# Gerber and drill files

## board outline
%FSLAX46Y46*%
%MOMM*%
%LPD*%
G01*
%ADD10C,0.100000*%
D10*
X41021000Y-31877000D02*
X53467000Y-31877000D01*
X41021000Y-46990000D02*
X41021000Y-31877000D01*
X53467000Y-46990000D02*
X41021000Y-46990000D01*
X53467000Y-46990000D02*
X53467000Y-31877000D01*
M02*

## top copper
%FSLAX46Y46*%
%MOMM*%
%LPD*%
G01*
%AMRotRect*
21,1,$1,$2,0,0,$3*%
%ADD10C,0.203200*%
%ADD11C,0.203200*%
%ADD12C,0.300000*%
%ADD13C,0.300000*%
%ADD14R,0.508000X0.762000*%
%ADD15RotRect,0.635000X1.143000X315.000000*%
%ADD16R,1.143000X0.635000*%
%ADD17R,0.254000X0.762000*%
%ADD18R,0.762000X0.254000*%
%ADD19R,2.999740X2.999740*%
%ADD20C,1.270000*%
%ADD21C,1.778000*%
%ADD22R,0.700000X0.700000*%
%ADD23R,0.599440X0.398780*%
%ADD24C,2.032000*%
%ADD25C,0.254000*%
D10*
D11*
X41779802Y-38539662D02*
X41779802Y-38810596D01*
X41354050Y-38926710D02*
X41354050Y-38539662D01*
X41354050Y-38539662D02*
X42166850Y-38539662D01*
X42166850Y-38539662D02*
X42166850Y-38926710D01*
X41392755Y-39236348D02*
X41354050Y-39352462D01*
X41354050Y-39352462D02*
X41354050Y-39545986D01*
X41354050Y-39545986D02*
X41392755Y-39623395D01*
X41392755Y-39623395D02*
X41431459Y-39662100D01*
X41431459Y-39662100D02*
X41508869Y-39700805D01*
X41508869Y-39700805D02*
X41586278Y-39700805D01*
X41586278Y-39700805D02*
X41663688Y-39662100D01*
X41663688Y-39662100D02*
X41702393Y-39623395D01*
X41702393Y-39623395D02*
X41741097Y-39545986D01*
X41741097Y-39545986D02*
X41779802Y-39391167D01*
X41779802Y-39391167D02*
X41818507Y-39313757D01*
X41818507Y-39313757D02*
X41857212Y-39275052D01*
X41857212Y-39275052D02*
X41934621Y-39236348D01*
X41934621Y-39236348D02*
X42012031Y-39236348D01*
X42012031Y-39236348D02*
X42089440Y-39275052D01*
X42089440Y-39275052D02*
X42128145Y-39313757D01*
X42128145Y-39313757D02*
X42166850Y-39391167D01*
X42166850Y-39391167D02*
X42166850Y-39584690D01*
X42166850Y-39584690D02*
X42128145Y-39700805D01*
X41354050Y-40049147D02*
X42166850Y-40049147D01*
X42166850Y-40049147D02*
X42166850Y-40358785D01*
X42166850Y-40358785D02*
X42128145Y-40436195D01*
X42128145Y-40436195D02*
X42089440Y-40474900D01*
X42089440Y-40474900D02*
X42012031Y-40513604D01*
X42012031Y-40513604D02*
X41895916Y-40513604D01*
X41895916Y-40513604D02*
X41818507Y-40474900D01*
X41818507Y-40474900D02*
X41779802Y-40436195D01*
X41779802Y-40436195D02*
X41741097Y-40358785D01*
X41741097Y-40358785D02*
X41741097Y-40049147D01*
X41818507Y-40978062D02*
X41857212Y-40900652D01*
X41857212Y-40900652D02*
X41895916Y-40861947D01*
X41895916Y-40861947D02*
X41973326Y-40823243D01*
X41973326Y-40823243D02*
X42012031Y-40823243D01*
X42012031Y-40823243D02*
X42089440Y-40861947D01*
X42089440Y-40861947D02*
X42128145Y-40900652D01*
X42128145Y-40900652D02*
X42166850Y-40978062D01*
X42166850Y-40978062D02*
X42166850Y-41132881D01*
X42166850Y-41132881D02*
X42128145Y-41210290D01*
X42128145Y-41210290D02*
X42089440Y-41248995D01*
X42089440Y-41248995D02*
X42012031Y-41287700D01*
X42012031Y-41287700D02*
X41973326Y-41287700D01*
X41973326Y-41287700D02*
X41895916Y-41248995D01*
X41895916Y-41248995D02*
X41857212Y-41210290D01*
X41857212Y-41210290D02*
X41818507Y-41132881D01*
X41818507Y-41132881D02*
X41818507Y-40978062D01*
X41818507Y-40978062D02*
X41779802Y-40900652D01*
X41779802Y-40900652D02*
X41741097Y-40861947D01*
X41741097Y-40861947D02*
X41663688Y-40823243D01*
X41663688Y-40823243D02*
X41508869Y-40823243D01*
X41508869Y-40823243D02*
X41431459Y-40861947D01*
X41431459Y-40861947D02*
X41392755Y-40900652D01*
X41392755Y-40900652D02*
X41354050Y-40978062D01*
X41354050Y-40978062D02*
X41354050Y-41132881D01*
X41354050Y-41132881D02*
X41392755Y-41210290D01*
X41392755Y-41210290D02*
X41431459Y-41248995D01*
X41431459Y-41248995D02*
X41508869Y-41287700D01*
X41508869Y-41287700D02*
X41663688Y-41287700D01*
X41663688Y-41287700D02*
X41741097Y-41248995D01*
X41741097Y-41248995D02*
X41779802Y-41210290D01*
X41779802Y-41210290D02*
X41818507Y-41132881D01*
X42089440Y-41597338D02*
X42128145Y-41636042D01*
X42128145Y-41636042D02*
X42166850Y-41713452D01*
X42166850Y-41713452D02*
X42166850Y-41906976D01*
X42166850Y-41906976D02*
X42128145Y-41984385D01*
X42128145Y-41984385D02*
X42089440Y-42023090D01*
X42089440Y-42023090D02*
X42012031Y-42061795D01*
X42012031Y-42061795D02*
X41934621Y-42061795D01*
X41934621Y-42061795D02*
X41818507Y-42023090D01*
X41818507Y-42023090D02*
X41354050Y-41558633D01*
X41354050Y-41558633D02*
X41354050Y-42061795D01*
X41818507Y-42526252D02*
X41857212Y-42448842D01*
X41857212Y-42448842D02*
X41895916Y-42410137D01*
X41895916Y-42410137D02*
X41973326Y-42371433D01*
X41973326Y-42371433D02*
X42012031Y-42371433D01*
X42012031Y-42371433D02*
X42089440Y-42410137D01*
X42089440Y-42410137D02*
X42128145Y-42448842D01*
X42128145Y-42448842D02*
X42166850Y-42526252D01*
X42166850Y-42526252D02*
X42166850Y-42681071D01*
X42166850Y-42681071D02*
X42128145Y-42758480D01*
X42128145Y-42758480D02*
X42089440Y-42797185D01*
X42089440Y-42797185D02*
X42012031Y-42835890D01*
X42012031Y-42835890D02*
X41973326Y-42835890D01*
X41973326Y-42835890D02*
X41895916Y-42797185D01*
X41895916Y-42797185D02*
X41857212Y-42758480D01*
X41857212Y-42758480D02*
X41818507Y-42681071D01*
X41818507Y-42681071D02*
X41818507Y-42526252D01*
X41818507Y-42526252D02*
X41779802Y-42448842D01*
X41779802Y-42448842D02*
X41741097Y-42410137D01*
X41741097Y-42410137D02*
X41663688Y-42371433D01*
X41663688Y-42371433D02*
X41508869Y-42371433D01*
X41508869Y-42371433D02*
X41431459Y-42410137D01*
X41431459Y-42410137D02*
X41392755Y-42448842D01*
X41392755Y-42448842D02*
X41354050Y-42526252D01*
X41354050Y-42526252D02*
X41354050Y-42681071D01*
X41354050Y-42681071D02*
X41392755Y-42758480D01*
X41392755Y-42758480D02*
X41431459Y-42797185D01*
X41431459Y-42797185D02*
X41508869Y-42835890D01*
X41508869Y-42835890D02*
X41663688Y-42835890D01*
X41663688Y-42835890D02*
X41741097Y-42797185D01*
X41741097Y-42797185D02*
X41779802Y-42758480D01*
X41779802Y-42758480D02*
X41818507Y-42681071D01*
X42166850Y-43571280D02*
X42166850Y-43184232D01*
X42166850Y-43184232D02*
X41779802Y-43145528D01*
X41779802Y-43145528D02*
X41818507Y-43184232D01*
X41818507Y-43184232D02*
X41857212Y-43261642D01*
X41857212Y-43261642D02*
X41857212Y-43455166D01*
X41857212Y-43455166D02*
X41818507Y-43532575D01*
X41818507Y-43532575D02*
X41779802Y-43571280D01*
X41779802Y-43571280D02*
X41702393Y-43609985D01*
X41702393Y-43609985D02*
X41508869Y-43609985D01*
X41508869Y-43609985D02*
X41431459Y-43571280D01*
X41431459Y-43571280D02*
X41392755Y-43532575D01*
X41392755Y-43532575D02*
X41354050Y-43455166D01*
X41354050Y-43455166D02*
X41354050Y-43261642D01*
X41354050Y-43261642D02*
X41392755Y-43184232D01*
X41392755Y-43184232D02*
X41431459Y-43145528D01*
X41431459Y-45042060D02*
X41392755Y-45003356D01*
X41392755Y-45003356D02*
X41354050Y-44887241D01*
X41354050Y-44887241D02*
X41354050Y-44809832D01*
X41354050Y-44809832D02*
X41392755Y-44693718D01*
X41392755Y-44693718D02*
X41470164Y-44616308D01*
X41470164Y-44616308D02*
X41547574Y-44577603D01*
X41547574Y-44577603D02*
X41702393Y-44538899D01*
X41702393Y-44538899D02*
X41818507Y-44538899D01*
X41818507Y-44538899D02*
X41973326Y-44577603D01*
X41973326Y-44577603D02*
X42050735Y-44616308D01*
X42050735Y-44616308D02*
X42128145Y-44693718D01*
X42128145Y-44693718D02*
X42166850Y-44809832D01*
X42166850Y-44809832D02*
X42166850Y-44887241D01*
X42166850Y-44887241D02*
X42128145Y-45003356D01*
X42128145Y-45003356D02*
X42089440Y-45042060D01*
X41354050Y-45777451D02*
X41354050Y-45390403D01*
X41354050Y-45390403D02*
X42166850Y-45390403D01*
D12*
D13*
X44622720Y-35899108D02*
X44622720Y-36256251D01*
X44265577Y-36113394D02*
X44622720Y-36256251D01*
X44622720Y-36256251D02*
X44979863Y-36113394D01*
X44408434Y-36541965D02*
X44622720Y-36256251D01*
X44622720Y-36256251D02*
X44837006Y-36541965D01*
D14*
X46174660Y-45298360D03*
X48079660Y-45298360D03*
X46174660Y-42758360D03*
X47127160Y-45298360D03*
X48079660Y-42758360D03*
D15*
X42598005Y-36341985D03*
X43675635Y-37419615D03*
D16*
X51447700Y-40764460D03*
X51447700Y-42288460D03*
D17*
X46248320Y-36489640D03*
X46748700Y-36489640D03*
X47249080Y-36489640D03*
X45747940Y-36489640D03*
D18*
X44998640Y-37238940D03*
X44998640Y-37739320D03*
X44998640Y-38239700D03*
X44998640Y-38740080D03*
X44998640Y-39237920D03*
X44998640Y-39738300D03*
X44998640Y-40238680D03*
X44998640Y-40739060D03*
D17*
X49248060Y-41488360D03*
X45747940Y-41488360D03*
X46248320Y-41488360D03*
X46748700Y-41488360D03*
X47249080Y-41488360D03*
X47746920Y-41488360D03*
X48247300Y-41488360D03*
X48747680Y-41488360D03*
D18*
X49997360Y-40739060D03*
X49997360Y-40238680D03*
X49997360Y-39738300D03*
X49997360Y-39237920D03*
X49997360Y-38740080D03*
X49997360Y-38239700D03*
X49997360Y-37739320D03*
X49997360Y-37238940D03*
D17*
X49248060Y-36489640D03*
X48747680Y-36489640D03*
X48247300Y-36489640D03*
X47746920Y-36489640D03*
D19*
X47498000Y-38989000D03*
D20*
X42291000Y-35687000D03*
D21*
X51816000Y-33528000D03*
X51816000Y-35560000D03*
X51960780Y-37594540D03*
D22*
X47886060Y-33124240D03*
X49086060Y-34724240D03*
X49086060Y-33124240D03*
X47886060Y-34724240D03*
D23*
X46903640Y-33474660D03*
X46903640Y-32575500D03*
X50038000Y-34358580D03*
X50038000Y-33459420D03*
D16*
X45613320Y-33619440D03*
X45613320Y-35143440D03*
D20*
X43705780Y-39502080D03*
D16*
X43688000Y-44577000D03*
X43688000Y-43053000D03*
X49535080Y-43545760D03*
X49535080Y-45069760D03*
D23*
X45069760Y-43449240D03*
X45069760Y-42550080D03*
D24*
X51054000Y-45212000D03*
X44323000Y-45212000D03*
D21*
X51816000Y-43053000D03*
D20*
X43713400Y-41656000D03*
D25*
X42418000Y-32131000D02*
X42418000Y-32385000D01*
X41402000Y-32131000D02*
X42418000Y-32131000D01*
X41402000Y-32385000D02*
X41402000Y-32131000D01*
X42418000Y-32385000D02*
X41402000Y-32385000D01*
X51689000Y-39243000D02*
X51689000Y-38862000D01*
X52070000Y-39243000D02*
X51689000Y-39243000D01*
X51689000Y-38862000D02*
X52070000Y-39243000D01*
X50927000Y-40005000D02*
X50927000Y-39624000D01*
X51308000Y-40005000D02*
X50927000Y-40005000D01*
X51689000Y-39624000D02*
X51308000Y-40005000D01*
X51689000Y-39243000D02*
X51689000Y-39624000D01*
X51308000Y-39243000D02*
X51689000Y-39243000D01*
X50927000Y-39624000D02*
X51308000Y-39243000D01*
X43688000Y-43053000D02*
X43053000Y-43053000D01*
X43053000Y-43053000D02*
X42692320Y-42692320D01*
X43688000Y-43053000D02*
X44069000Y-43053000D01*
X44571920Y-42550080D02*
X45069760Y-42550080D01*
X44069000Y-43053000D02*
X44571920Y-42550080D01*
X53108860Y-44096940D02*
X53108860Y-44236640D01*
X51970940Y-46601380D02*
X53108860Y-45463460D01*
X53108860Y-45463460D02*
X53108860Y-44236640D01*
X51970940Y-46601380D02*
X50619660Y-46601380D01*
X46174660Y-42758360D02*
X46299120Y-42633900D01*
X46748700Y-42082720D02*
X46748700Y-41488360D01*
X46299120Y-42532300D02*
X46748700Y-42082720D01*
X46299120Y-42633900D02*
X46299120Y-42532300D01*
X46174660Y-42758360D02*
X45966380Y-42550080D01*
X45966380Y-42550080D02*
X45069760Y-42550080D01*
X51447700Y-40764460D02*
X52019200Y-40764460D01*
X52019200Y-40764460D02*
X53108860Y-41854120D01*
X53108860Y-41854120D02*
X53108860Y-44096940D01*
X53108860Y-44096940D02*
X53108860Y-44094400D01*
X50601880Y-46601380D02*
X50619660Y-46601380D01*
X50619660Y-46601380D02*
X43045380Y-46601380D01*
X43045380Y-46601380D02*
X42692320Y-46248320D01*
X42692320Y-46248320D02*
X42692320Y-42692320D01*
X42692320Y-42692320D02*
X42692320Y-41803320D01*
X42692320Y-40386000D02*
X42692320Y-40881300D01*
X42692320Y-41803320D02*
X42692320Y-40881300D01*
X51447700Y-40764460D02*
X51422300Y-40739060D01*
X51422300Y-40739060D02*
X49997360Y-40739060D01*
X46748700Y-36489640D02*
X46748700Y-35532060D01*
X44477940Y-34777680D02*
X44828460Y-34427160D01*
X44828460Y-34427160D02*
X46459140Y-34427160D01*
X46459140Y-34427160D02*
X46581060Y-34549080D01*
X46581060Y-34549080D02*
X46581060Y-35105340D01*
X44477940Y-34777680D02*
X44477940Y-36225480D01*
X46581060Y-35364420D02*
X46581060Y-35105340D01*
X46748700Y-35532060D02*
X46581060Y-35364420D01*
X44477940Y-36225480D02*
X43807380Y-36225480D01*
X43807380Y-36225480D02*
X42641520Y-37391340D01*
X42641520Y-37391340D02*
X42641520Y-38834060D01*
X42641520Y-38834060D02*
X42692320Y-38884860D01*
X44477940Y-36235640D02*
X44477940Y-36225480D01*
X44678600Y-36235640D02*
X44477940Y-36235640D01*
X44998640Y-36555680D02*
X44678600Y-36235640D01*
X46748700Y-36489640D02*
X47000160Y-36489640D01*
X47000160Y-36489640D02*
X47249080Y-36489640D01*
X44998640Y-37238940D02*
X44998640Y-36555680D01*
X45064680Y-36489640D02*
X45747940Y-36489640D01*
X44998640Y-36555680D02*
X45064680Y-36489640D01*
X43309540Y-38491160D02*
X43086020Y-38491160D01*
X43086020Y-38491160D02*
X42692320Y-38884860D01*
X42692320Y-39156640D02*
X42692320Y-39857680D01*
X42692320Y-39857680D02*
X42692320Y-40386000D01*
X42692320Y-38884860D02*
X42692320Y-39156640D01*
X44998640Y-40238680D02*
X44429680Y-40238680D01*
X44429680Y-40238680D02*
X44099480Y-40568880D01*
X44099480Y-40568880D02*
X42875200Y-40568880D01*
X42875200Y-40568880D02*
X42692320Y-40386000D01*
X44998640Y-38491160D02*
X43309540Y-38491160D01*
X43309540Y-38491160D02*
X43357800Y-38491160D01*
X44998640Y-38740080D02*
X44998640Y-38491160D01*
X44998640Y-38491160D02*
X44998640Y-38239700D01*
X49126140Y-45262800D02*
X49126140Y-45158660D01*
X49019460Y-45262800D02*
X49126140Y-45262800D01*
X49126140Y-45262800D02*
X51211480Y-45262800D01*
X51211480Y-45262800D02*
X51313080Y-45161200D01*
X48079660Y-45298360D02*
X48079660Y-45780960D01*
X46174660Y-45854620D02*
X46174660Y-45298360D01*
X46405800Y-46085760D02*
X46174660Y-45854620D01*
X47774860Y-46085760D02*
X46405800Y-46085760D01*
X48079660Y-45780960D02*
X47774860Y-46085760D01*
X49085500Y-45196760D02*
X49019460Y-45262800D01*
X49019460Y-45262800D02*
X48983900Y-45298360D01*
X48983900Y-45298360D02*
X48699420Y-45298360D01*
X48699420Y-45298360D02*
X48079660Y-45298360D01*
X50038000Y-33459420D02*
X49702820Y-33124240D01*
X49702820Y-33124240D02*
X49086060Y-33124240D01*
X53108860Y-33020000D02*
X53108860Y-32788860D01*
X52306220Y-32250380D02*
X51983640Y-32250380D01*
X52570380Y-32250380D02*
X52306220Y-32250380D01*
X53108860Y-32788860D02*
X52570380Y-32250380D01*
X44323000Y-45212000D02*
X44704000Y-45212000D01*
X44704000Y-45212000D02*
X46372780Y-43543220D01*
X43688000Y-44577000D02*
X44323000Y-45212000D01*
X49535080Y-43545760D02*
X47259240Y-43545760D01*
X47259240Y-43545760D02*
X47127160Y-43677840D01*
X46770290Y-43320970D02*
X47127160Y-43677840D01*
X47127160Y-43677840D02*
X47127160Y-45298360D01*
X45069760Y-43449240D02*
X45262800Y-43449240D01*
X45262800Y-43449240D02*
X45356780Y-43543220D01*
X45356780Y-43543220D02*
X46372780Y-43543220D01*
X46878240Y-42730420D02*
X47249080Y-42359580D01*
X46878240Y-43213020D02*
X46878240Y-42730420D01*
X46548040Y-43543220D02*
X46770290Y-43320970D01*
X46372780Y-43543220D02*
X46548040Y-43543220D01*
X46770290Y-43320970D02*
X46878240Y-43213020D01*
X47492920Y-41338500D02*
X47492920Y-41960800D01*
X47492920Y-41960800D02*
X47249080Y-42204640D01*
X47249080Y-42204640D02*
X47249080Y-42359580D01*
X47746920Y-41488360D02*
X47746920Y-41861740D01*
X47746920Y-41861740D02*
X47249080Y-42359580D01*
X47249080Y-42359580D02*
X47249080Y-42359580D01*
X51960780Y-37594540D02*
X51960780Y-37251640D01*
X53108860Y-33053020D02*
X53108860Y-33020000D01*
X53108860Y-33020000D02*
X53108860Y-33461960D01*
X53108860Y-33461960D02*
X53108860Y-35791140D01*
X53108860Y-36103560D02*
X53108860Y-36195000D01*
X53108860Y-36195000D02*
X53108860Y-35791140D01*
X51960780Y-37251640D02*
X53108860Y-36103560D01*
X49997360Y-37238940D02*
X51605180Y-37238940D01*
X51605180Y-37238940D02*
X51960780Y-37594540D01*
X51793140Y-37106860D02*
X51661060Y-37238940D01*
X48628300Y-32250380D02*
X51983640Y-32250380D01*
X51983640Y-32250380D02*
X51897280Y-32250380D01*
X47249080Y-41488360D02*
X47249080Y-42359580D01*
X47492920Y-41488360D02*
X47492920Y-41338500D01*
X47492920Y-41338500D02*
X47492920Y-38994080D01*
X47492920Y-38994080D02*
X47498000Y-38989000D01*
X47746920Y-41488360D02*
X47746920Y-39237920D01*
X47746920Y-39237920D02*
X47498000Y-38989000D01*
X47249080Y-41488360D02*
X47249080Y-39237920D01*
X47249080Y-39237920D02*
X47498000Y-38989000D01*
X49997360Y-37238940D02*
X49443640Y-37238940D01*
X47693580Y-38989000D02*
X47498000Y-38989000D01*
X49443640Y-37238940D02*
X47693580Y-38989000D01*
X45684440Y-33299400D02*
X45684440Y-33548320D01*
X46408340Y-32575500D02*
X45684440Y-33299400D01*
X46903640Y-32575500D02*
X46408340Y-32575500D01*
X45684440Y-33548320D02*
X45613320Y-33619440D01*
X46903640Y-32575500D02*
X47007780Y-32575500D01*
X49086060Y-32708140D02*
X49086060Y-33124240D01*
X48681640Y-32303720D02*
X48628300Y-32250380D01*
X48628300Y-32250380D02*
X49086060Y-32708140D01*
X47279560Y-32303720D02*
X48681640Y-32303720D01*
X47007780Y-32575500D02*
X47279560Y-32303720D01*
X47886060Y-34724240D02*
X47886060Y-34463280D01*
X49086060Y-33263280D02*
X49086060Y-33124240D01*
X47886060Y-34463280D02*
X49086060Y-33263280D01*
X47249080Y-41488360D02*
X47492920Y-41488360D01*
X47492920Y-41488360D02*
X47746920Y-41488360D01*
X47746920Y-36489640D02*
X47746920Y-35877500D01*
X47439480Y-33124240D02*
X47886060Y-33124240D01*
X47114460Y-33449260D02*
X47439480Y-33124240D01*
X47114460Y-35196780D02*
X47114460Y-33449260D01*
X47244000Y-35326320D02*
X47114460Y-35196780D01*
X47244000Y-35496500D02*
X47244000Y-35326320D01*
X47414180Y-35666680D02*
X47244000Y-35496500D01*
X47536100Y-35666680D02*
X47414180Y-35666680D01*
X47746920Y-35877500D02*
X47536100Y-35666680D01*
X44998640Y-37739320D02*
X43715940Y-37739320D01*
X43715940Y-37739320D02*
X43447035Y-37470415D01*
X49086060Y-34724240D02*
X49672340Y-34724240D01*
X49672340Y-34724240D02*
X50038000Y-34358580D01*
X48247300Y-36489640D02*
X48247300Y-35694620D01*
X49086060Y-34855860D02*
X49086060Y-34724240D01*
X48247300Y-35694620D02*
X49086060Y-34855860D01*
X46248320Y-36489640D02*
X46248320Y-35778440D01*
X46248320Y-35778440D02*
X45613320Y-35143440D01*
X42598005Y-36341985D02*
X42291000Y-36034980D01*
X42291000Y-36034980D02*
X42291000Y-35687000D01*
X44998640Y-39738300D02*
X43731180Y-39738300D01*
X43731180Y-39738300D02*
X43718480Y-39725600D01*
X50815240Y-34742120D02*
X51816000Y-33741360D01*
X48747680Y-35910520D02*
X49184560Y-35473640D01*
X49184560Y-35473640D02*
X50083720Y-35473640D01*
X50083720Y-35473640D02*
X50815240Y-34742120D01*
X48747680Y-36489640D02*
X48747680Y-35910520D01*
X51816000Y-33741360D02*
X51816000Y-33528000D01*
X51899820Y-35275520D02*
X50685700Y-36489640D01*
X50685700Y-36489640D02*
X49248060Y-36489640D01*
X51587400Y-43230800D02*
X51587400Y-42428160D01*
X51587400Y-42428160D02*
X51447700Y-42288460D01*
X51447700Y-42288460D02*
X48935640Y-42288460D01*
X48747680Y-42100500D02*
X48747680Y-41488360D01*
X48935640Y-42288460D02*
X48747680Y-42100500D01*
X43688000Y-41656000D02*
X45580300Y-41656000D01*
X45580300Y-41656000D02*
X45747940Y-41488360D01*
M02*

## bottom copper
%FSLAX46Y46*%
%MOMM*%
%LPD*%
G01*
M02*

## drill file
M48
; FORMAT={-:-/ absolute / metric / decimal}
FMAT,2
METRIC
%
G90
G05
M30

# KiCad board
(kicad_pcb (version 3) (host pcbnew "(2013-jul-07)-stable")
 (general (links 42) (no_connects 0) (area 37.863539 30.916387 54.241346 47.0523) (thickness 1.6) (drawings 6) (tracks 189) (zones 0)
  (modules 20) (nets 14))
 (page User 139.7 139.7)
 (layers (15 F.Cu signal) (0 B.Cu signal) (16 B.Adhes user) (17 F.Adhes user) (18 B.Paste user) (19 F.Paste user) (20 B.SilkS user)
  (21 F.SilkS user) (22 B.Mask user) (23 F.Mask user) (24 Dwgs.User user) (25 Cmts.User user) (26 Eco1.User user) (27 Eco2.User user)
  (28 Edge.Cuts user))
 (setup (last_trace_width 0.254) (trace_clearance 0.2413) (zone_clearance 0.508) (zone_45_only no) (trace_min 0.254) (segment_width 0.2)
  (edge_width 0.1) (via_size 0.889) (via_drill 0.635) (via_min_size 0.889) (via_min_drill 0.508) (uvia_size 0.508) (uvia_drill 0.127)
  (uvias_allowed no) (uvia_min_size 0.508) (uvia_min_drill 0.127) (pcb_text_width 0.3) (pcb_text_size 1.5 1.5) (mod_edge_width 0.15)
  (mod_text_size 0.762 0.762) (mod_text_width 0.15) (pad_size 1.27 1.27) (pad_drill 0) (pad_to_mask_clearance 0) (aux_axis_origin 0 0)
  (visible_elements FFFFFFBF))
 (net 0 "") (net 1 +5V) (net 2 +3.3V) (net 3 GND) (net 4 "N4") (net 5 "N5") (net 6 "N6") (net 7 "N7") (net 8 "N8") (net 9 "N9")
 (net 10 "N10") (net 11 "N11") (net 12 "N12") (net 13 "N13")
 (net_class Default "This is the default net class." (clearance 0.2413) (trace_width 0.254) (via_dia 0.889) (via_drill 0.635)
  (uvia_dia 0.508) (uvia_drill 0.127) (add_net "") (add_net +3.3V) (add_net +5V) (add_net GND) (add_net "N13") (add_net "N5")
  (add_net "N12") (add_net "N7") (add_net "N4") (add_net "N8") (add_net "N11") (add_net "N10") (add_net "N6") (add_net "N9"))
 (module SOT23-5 (layer F.Cu) (at 47.12716 44.02836)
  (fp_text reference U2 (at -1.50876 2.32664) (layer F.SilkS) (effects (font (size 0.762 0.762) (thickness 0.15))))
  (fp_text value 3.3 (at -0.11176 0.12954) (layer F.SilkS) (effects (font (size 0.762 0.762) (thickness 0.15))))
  (pad 1 smd rect (at -0.9525 1.27) (size 0.508 0.762) (layers F.Cu F.Paste F.Mask) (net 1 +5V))
  (pad 3 smd rect (at 0.9525 1.27) (size 0.508 0.762) (layers F.Cu F.Paste F.Mask) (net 1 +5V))
  (pad 5 smd rect (at -0.9525 -1.27) (size 0.508 0.762) (layers F.Cu F.Paste F.Mask) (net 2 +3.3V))
  (pad 2 smd rect (at 0 1.27) (size 0.508 0.762) (layers F.Cu F.Paste F.Mask) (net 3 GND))
  (pad 4 smd rect (at 0.9525 -1.27) (size 0.508 0.762) (layers F.Cu F.Paste F.Mask)))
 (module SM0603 (layer F.Cu) (at 43.13682 36.8808 315)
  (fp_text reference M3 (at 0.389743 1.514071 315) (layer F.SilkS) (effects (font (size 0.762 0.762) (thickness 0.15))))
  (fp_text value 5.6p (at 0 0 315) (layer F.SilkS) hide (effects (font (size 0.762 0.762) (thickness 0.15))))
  (pad 1 smd rect (at -0.762 0 315) (size 0.635 1.143) (layers F.Cu F.Paste F.Mask) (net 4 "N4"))
  (pad 2 smd rect (at 0.762 0 315) (size 0.635 1.143) (layers F.Cu F.Paste F.Mask) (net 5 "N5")))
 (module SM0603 (layer F.Cu) (at 51.4477 41.52646 270)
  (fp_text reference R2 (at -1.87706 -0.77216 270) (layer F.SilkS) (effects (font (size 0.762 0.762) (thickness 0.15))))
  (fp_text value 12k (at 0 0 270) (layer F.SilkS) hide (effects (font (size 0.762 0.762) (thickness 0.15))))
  (pad 1 smd rect (at -0.762 0 270) (size 0.635 1.143) (layers F.Cu F.Paste F.Mask) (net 2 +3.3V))
  (pad 2 smd rect (at 0.762 0 270) (size 0.635 1.143) (layers F.Cu F.Paste F.Mask) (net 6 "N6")))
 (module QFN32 (layer F.Cu) (at 47.498 38.989)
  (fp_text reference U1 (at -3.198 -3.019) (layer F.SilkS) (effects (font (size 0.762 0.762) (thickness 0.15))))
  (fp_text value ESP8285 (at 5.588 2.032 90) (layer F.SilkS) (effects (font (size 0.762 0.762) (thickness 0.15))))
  (pad 31 smd rect (at -1.24968 -2.49936) (size 0.254 0.762) (layers F.Cu F.Paste F.Mask) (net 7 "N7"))
  (pad 30 smd rect (at -0.7493 -2.49936) (size 0.254 0.762) (layers F.Cu F.Paste F.Mask) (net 2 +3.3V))
  (pad 29 smd rect (at -0.24892 -2.49936) (size 0.254 0.762) (layers F.Cu F.Paste F.Mask) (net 2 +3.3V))
  (pad 32 smd rect (at -1.75006 -2.49936) (size 0.254 0.762) (layers F.Cu F.Paste F.Mask) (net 2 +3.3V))
  (pad 1 smd rect (at -2.49936 -1.75006 90) (size 0.254 0.762) (layers F.Cu F.Paste F.Mask) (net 2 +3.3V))
  (pad 2 smd rect (at -2.49936 -1.24968 90) (size 0.254 0.762) (layers F.Cu F.Paste F.Mask) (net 5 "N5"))
  (pad 3 smd rect (at -2.49936 -0.7493 90) (size 0.254 0.762) (layers F.Cu F.Paste F.Mask) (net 2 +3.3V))
  (pad 4 smd rect (at -2.49936 -0.24892 90) (size 0.254 0.762) (layers F.Cu F.Paste F.Mask) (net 2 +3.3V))
  (pad 5 smd rect (at -2.49936 0.24892 90) (size 0.254 0.762) (layers F.Cu F.Paste F.Mask))
  (pad 6 smd rect (at -2.49936 0.7493 90) (size 0.254 0.762) (layers F.Cu F.Paste F.Mask) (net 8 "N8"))
  (pad 7 smd rect (at -2.49936 1.24968 90) (size 0.254 0.762) (layers F.Cu F.Paste F.Mask) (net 2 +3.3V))
  (pad 8 smd rect (at -2.49936 1.75006 90) (size 0.254 0.762) (layers F.Cu F.Paste F.Mask))
  (pad 16 smd rect (at 1.75006 2.49936) (size 0.254 0.762) (layers F.Cu F.Paste F.Mask))
  (pad 9 smd rect (at -1.75006 2.49936) (size 0.254 0.762) (layers F.Cu F.Paste F.Mask) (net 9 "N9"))
  (pad 10 smd rect (at -1.24968 2.49936) (size 0.254 0.762) (layers F.Cu F.Paste F.Mask))
  (pad 11 smd rect (at -0.7493 2.49936) (size 0.254 0.762) (layers F.Cu F.Paste F.Mask) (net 2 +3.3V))
  (pad 12 smd rect (at -0.24892 2.49936) (size 0.254 0.762) (layers F.Cu F.Paste F.Mask) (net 3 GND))
  (pad 13 smd rect (at 0.24892 2.49936) (size 0.254 0.762) (layers F.Cu F.Paste F.Mask) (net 3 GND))
  (pad 14 smd rect (at 0.7493 2.49936) (size 0.254 0.762) (layers F.Cu F.Paste F.Mask))
  (pad 15 smd rect (at 1.24968 2.49936) (size 0.254 0.762) (layers F.Cu F.Paste F.Mask) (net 6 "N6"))
  (pad 17 smd rect (at 2.49936 1.75006 90) (size 0.254 0.762) (layers F.Cu F.Paste F.Mask) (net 2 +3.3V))
  (pad 18 smd rect (at 2.49936 1.24968 90) (size 0.254 0.762) (layers F.Cu F.Paste F.Mask))
  (pad 19 smd rect (at 2.49936 0.7493 90) (size 0.254 0.762) (layers F.Cu F.Paste F.Mask))
  (pad 20 smd rect (at 2.49936 0.24892 90) (size 0.254 0.762) (layers F.Cu F.Paste F.Mask))
  (pad 21 smd rect (at 2.49936 -0.24892 90) (size 0.254 0.762) (layers F.Cu F.Paste F.Mask))
  (pad 22 smd rect (at 2.49936 -0.7493 90) (size 0.254 0.762) (layers F.Cu F.Paste F.Mask))
  (pad 23 smd rect (at 2.49936 -1.24968 90) (size 0.254 0.762) (layers F.Cu F.Paste F.Mask))
  (pad 24 smd rect (at 2.49936 -1.75006 90) (size 0.254 0.762) (layers F.Cu F.Paste F.Mask) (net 3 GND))
  (pad 25 smd rect (at 1.75006 -2.49936) (size 0.254 0.762) (layers F.Cu F.Paste F.Mask) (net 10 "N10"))
  (pad 26 smd rect (at 1.24968 -2.49936) (size 0.254 0.762) (layers F.Cu F.Paste F.Mask) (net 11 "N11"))
  (pad 27 smd rect (at 0.7493 -2.49936) (size 0.254 0.762) (layers F.Cu F.Paste F.Mask) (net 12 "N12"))
  (pad 28 smd rect (at 0.24892 -2.49936) (size 0.254 0.762) (layers F.Cu F.Paste F.Mask) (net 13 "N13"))
  (pad 33 smd rect (at 0 0) (size 2.99974 2.99974) (layers F.Cu F.Paste F.Mask) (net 3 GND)))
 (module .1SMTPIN (layer F.Cu) (at 42.291 35.687)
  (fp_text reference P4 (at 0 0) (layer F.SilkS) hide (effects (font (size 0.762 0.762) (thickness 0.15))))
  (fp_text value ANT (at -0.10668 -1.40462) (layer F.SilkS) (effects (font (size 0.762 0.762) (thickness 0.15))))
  (pad 1 smd circle (at 0 0) (size 1.27 1.27) (layers F.Cu F.Paste F.Mask) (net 4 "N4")))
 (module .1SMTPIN (layer F.Cu) (at 51.816 33.528)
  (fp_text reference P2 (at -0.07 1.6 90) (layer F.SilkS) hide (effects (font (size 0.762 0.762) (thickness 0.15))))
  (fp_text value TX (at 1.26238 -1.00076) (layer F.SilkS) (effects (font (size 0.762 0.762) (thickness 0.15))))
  (pad 1 smd circle (at 0 0) (size 1.778 1.778) (layers F.Cu F.Paste F.Mask) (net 11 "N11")))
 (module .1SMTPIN (layer F.Cu) (at 51.816 35.56)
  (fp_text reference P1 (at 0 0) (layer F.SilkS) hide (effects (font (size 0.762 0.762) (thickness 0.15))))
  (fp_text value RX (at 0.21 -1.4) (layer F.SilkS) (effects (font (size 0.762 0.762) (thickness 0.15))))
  (pad 1 smd circle (at 0 0) (size 1.778 1.778) (layers F.Cu F.Paste F.Mask) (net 10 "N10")))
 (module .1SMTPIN (layer F.Cu) (at 51.96078 37.59454)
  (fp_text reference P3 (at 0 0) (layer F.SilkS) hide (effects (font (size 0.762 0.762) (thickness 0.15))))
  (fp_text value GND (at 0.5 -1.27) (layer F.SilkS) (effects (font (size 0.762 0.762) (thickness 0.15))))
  (pad 1 smd circle (at 0 0) (size 1.778 1.778) (layers F.Cu F.Paste F.Mask) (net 3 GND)))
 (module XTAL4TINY (layer F.Cu) (at 48.48606 33.92424 270)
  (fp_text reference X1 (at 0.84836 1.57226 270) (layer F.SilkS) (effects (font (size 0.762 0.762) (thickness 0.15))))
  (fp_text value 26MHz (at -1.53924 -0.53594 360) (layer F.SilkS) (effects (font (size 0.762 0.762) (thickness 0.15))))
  (pad 1 smd rect (at -0.8 0.6 270) (size 0.7 0.7) (layers F.Cu F.Paste F.Mask) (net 13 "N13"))
  (pad 2 smd rect (at 0.8 -0.6 270) (size 0.7 0.7) (layers F.Cu F.Paste F.Mask) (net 12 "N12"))
  (pad 3 smd rect (at -0.8 -0.6 270) (size 0.7 0.7) (layers F.Cu F.Paste F.Mask) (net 3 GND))
  (pad 4 smd rect (at 0.8 0.6 270) (size 0.7 0.7) (layers F.Cu F.Paste F.Mask) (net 3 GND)))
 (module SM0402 (layer F.Cu) (at 46.90364 33.02508 90)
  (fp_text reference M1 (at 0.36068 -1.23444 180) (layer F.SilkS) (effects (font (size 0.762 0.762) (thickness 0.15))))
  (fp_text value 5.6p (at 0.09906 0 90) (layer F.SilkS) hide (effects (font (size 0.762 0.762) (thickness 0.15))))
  (pad 1 smd rect (at -0.44958 0 90) (size 0.39878 0.59944) (layers F.Cu F.Paste F.Mask) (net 13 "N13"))
  (pad 2 smd rect (at 0.44958 0 90) (size 0.39878 0.59944) (layers F.Cu F.Paste F.Mask) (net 3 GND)))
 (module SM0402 (layer F.Cu) (at 50.038 33.909 90)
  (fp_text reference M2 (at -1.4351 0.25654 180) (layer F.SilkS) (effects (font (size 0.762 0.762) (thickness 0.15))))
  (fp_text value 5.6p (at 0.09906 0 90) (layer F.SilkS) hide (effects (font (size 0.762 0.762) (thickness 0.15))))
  (pad 1 smd rect (at -0.44958 0 90) (size 0.39878 0.59944) (layers F.Cu F.Paste F.Mask) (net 12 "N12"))
  (pad 2 smd rect (at 0.44958 0 90) (size 0.39878 0.59944) (layers F.Cu F.Paste F.Mask) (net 3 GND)))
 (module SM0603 (layer F.Cu) (at 45.61332 34.38144 270)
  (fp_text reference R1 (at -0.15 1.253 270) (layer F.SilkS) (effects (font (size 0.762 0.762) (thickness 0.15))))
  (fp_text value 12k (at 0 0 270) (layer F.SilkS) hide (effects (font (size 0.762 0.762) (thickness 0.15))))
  (pad 1 smd rect (at -0.762 0 270) (size 0.635 1.143) (layers F.Cu F.Paste F.Mask) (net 3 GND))
  (pad 2 smd rect (at 0.762 0 270) (size 0.635 1.143) (layers F.Cu F.Paste F.Mask) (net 7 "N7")))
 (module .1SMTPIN (layer F.Cu) (at 43.70324 39.50208)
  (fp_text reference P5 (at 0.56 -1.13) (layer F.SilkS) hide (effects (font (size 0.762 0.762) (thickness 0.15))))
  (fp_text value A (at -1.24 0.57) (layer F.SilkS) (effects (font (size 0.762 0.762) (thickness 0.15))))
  (pad 1 smd circle (at 0.00254 0) (size 1.27 1.27) (layers F.Cu F.Paste F.Mask) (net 8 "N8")))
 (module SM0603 (layer F.Cu) (at 43.688 43.815 90)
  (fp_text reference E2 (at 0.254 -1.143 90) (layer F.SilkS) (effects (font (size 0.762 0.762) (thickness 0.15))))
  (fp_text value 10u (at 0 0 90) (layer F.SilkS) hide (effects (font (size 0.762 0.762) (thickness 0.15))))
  (pad 1 smd rect (at -0.762 0 90) (size 0.635 1.143) (layers F.Cu F.Paste F.Mask) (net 3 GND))
  (pad 2 smd rect (at 0.762 0 90) (size 0.635 1.143) (layers F.Cu F.Paste F.Mask) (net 2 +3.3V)))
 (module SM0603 (layer F.Cu) (at 49.53508 44.30776 270)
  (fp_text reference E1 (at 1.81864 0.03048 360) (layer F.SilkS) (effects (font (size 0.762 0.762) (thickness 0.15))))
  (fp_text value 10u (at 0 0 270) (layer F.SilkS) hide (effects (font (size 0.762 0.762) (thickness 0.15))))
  (pad 1 smd rect (at -0.762 0 270) (size 0.635 1.143) (layers F.Cu F.Paste F.Mask) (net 3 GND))
  (pad 2 smd rect (at 0.762 0 270) (size 0.635 1.143) (layers F.Cu F.Paste F.Mask) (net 1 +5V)))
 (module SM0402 (layer F.Cu) (at 45.06976 42.99966 90)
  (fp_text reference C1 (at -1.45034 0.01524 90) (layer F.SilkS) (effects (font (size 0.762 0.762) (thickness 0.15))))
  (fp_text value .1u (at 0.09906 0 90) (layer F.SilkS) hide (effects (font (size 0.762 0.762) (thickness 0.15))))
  (pad 1 smd rect (at -0.44958 0 90) (size 0.39878 0.59944) (layers F.Cu F.Paste F.Mask) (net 3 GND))
  (pad 2 smd rect (at 0.44958 0 90) (size 0.39878 0.59944) (layers F.Cu F.Paste F.Mask) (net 2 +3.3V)))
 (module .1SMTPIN (layer F.Cu) (at 51.054 45.212)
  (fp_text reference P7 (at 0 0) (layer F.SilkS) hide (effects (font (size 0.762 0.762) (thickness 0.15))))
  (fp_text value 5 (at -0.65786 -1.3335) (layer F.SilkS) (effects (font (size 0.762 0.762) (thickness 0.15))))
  (pad 1 smd circle (at 0 0) (size 2.032 2.032) (layers F.Cu F.Paste F.Mask) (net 1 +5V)))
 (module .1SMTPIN (layer F.Cu) (at 44.323 45.212)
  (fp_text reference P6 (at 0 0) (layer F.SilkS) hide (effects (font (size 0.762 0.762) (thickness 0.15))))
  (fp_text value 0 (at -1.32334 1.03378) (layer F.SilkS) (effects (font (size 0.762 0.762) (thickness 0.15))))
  (pad 1 smd circle (at 0 0) (size 2.032 2.032) (layers F.Cu F.Paste F.Mask) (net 3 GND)))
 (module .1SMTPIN (layer F.Cu) (at 51.816 43.053)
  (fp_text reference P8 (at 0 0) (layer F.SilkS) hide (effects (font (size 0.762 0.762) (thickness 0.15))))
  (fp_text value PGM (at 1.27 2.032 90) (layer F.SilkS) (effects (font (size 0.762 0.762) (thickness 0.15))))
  (pad 1 smd circle (at 0 0) (size 1.778 1.778) (layers F.Cu F.Paste F.Mask) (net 6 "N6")))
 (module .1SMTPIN (layer F.Cu) (at 43.688 41.656)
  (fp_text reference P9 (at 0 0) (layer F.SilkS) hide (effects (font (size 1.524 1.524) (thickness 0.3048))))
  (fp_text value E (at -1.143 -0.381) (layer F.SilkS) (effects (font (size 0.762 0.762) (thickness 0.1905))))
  (pad 1 smd circle (at 0.0254 0) (size 1.27 1.27) (layers F.Cu F.Paste F.Mask) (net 9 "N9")))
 (gr_line (start 41.021 31.877) (end 53.467 31.877) (angle 90) (layer Edge.Cuts) (width 0.1))
 (gr_line (start 41.021 46.99) (end 41.021 31.877) (angle 90) (layer Edge.Cuts) (width 0.1))
 (gr_line (start 53.467 46.99) (end 41.021 46.99) (angle 90) (layer Edge.Cuts) (width 0.1))
 (gr_line (start 53.467 46.99) (end 53.467 31.877) (angle 90) (layer Edge.Cuts) (width 0.1))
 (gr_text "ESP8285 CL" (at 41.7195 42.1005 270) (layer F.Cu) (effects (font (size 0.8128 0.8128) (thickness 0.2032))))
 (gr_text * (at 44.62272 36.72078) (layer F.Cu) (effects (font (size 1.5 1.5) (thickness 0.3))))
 (segment (start 42.418 32.131) (end 42.418 32.385) (width 0.254) (layer F.Cu) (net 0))
 (segment (start 41.402 32.131) (end 42.418 32.131) (width 0.254) (layer F.Cu) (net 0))
 (segment (start 41.402 32.385) (end 41.402 32.131) (width 0.254) (layer F.Cu) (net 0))
 (segment (start 42.418 32.385) (end 41.402 32.385) (width 0.254) (layer F.Cu) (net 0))
 (segment (start 51.689 39.243) (end 51.689 38.862) (width 0.254) (layer F.Cu) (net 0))
 (segment (start 52.07 39.243) (end 51.689 39.243) (width 0.254) (layer F.Cu) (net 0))
 (segment (start 51.689 38.862) (end 52.07 39.243) (width 0.254) (layer F.Cu) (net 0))
 (segment (start 50.927 40.005) (end 50.927 39.624) (width 0.254) (layer F.Cu) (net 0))
 (segment (start 51.308 40.005) (end 50.927 40.005) (width 0.254) (layer F.Cu) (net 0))
 (segment (start 51.689 39.624) (end 51.308 40.005) (width 0.254) (layer F.Cu) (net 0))
 (segment (start 51.689 39.243) (end 51.689 39.624) (width 0.254) (layer F.Cu) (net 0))
 (segment (start 51.308 39.243) (end 51.689 39.243) (width 0.254) (layer F.Cu) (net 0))
 (segment (start 50.927 39.624) (end 51.308 39.243) (width 0.254) (layer F.Cu) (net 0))
 (segment (start 43.688 43.053) (end 43.053 43.053) (width 0.254) (layer F.Cu) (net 2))
 (segment (start 43.053 43.053) (end 42.69232 42.69232) (width 0.254) (layer F.Cu) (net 2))
 (segment (start 43.688 43.053) (end 44.069 43.053) (width 0.254) (layer F.Cu) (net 2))
 (segment (start 44.57192 42.55008) (end 45.06976 42.55008) (width 0.254) (layer F.Cu) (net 2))
 (segment (start 44.069 43.053) (end 44.57192 42.55008) (width 0.254) (layer F.Cu) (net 2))
 (segment (start 53.10886 44.09694) (end 53.10886 44.23664) (width 0.254) (layer F.Cu) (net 2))
 (segment (start 51.97094 46.60138) (end 53.10886 45.46346) (width 0.254) (layer F.Cu) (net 2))
 (segment (start 53.10886 45.46346) (end 53.10886 44.23664) (width 0.254) (layer F.Cu) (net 2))
 (segment (start 51.97094 46.60138) (end 50.61966 46.60138) (width 0.254) (layer F.Cu) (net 2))
 (segment (start 46.17466 42.75836) (end 46.29912 42.6339) (width 0.254) (layer F.Cu) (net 2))
 (segment (start 46.7487 42.08272) (end 46.7487 41.48836) (width 0.254) (layer F.Cu) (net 2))
 (segment (start 46.29912 42.5323) (end 46.7487 42.08272) (width 0.254) (layer F.Cu) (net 2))
 (segment (start 46.29912 42.6339) (end 46.29912 42.5323) (width 0.254) (layer F.Cu) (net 2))
 (segment (start 46.17466 42.75836) (end 45.96638 42.55008) (width 0.254) (layer F.Cu) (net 2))
 (segment (start 45.96638 42.55008) (end 45.06976 42.55008) (width 0.254) (layer F.Cu) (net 2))
 (segment (start 51.4477 40.76446) (end 52.0192 40.76446) (width 0.254) (layer F.Cu) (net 2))
 (segment (start 52.0192 40.76446) (end 53.10886 41.85412) (width 0.254) (layer F.Cu) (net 2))
 (segment (start 53.10886 41.85412) (end 53.10886 44.09694) (width 0.254) (layer F.Cu) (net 2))
 (segment (start 53.10886 44.09694) (end 53.10886 44.0944) (width 0.254) (layer F.Cu) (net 2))
 (segment (start 50.60188 46.60138) (end 50.61966 46.60138) (width 0.254) (layer F.Cu) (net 2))
 (segment (start 50.61966 46.60138) (end 43.04538 46.60138) (width 0.254) (layer F.Cu) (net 2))
 (segment (start 43.04538 46.60138) (end 42.69232 46.24832) (width 0.254) (layer F.Cu) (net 2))
 (segment (start 42.69232 46.24832) (end 42.69232 42.69232) (width 0.254) (layer F.Cu) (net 2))
 (segment (start 42.69232 42.69232) (end 42.69232 41.80332) (width 0.254) (layer F.Cu) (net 2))
 (segment (start 42.69232 40.386) (end 42.69232 40.8813) (width 0.254) (layer F.Cu) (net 2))
 (segment (start 42.69232 41.80332) (end 42.69232 40.8813) (width 0.254) (layer F.Cu) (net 2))
 (segment (start 51.4477 40.76446) (end 51.4223 40.73906) (width 0.254) (layer F.Cu) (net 2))
 (segment (start 51.4223 40.73906) (end 49.99736 40.73906) (width 0.254) (layer F.Cu) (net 2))
 (segment (start 46.7487 36.48964) (end 46.7487 35.53206) (width 0.254) (layer F.Cu) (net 2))
 (segment (start 44.47794 34.77768) (end 44.82846 34.42716) (width 0.254) (layer F.Cu) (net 2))
 (segment (start 44.82846 34.42716) (end 46.45914 34.42716) (width 0.254) (layer F.Cu) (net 2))
 (segment (start 46.45914 34.42716) (end 46.58106 34.54908) (width 0.254) (layer F.Cu) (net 2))
 (segment (start 46.58106 34.54908) (end 46.58106 35.10534) (width 0.254) (layer F.Cu) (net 2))
 (segment (start 44.47794 34.77768) (end 44.47794 36.22548) (width 0.254) (layer F.Cu) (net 2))
 (segment (start 46.58106 35.36442) (end 46.58106 35.10534) (width 0.254) (layer F.Cu) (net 2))
 (segment (start 46.7487 35.53206) (end 46.58106 35.36442) (width 0.254) (layer F.Cu) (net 2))
 (segment (start 44.47794 36.22548) (end 43.80738 36.22548) (width 0.254) (layer F.Cu) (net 2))
 (segment (start 43.80738 36.22548) (end 42.64152 37.39134) (width 0.254) (layer F.Cu) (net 2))
 (segment (start 42.64152 37.39134) (end 42.64152 38.83406) (width 0.254) (layer F.Cu) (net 2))
 (segment (start 42.64152 38.83406) (end 42.69232 38.88486) (width 0.254) (layer F.Cu) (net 2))
 (segment (start 44.47794 36.23564) (end 44.47794 36.22548) (width 0.254) (layer F.Cu) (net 2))
 (segment (start 44.6786 36.23564) (end 44.47794 36.23564) (width 0.254) (layer F.Cu) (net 2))
 (segment (start 44.99864 36.55568) (end 44.6786 36.23564) (width 0.254) (layer F.Cu) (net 2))
 (segment (start 46.7487 36.48964) (end 47.00016 36.48964) (width 0.254) (layer F.Cu) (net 2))
 (segment (start 47.00016 36.48964) (end 47.24908 36.48964) (width 0.254) (layer F.Cu) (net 2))
 (segment (start 44.99864 37.23894) (end 44.99864 36.55568) (width 0.254) (layer F.Cu) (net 2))
 (segment (start 45.06468 36.48964) (end 45.74794 36.48964) (width 0.254) (layer F.Cu) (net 2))
 (segment (start 44.99864 36.55568) (end 45.06468 36.48964) (width 0.254) (layer F.Cu) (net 2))
 (segment (start 43.30954 38.49116) (end 43.08602 38.49116) (width 0.254) (layer F.Cu) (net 2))
 (segment (start 43.08602 38.49116) (end 42.69232 38.88486) (width 0.254) (layer F.Cu) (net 2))
 (segment (start 42.69232 39.15664) (end 42.69232 39.85768) (width 0.254) (layer F.Cu) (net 2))
 (segment (start 42.69232 39.85768) (end 42.69232 40.386) (width 0.254) (layer F.Cu) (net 2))
 (segment (start 42.69232 38.88486) (end 42.69232 39.15664) (width 0.254) (layer F.Cu) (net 2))
 (segment (start 44.99864 40.23868) (end 44.42968 40.23868) (width 0.254) (layer F.Cu) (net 2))
 (segment (start 44.42968 40.23868) (end 44.09948 40.56888) (width 0.254) (layer F.Cu) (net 2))
 (segment (start 44.09948 40.56888) (end 42.8752 40.56888) (width 0.254) (layer F.Cu) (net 2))
 (segment (start 42.8752 40.56888) (end 42.69232 40.386) (width 0.254) (layer F.Cu) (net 2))
 (segment (start 44.99864 38.49116) (end 43.30954 38.49116) (width 0.254) (layer F.Cu) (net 2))
 (segment (start 43.30954 38.49116) (end 43.3578 38.49116) (width 0.254) (layer F.Cu) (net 2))
 (segment (start 44.99864 38.74008) (end 44.99864 38.49116) (width 0.254) (layer F.Cu) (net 2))
 (segment (start 44.99864 38.49116) (end 44.99864 38.2397) (width 0.254) (layer F.Cu) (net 2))
 (segment (start 49.12614 45.2628) (end 49.12614 45.15866) (width 0.254) (layer F.Cu) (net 1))
 (segment (start 49.01946 45.2628) (end 49.12614 45.2628) (width 0.254) (layer F.Cu) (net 1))
 (segment (start 49.12614 45.2628) (end 51.21148 45.2628) (width 0.254) (layer F.Cu) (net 1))
 (segment (start 51.21148 45.2628) (end 51.31308 45.1612) (width 0.254) (layer F.Cu) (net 1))
 (segment (start 48.07966 45.29836) (end 48.07966 45.78096) (width 0.254) (layer F.Cu) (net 1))
 (segment (start 46.17466 45.85462) (end 46.17466 45.29836) (width 0.254) (layer F.Cu) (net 1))
 (segment (start 46.4058 46.08576) (end 46.17466 45.85462) (width 0.254) (layer F.Cu) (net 1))
 (segment (start 47.77486 46.08576) (end 46.4058 46.08576) (width 0.254) (layer F.Cu) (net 1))
 (segment (start 48.07966 45.78096) (end 47.77486 46.08576) (width 0.254) (layer F.Cu) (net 1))
 (segment (start 49.0855 45.19676) (end 49.01946 45.2628) (width 0.254) (layer F.Cu) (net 1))
 (segment (start 49.01946 45.2628) (end 48.9839 45.29836) (width 0.254) (layer F.Cu) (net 1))
 (segment (start 48.9839 45.29836) (end 48.69942 45.29836) (width 0.254) (layer F.Cu) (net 1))
 (segment (start 48.69942 45.29836) (end 48.07966 45.29836) (width 0.254) (layer F.Cu) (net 1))
 (segment (start 50.038 33.45942) (end 49.70282 33.12424) (width 0.254) (layer F.Cu) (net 3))
 (segment (start 49.70282 33.12424) (end 49.08606 33.12424) (width 0.254) (layer F.Cu) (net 3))
 (segment (start 53.10886 33.02) (end 53.10886 32.78886) (width 0.254) (layer F.Cu) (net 3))
 (segment (start 52.30622 32.25038) (end 51.98364 32.25038) (width 0.254) (layer F.Cu) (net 3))
 (segment (start 52.57038 32.25038) (end 52.30622 32.25038) (width 0.254) (layer F.Cu) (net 3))
 (segment (start 53.10886 32.78886) (end 52.57038 32.25038) (width 0.254) (layer F.Cu) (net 3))
 (segment (start 44.323 45.212) (end 44.704 45.212) (width 0.254) (layer F.Cu) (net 3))
 (segment (start 44.704 45.212) (end 46.37278 43.54322) (width 0.254) (layer F.Cu) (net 3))
 (segment (start 43.688 44.577) (end 44.323 45.212) (width 0.254) (layer F.Cu) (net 3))
 (segment (start 49.53508 43.54576) (end 47.25924 43.54576) (width 0.254) (layer F.Cu) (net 3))
 (segment (start 47.25924 43.54576) (end 47.12716 43.67784) (width 0.254) (layer F.Cu) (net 3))
 (segment (start 46.77029 43.32097) (end 47.12716 43.67784) (width 0.254) (layer F.Cu) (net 3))
 (segment (start 47.12716 43.67784) (end 47.12716 45.29836) (width 0.254) (layer F.Cu) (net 3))
 (segment (start 45.06976 43.44924) (end 45.2628 43.44924) (width 0.254) (layer F.Cu) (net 3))
 (segment (start 45.2628 43.44924) (end 45.35678 43.54322) (width 0.254) (layer F.Cu) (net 3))
 (segment (start 45.35678 43.54322) (end 46.37278 43.54322) (width 0.254) (layer F.Cu) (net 3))
 (segment (start 46.87824 42.73042) (end 47.24908 42.35958) (width 0.254) (layer F.Cu) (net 3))
 (segment (start 46.87824 43.21302) (end 46.87824 42.73042) (width 0.254) (layer F.Cu) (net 3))
 (segment (start 46.54804 43.54322) (end 46.77029 43.32097) (width 0.254) (layer F.Cu) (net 3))
 (segment (start 46.37278 43.54322) (end 46.54804 43.54322) (width 0.254) (layer F.Cu) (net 3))
 (segment (start 46.77029 43.32097) (end 46.87824 43.21302) (width 0.254) (layer F.Cu) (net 3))
 (segment (start 47.49292 41.3385) (end 47.49292 41.9608) (width 0.254) (layer F.Cu) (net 3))
 (segment (start 47.49292 41.9608) (end 47.24908 42.20464) (width 0.254) (layer F.Cu) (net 3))
 (segment (start 47.24908 42.20464) (end 47.24908 42.35958) (width 0.254) (layer F.Cu) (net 3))
 (segment (start 47.74692 41.48836) (end 47.74692 41.86174) (width 0.254) (layer F.Cu) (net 3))
 (segment (start 47.74692 41.86174) (end 47.24908 42.35958) (width 0.254) (layer F.Cu) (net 3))
 (segment (start 47.24908 42.35958) (end 47.24908 42.35958) (width 0.254) (layer F.Cu) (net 3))
 (segment (start 51.96078 37.59454) (end 51.96078 37.25164) (width 0.254) (layer F.Cu) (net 3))
 (segment (start 53.10886 33.05302) (end 53.10886 33.02) (width 0.254) (layer F.Cu) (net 3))
 (segment (start 53.10886 33.02) (end 53.10886 33.46196) (width 0.254) (layer F.Cu) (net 3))
 (segment (start 53.10886 33.46196) (end 53.10886 35.79114) (width 0.254) (layer F.Cu) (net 3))
 (segment (start 53.10886 36.10356) (end 53.10886 36.195) (width 0.254) (layer F.Cu) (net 3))
 (segment (start 53.10886 36.195) (end 53.10886 35.79114) (width 0.254) (layer F.Cu) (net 3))
 (segment (start 51.96078 37.25164) (end 53.10886 36.10356) (width 0.254) (layer F.Cu) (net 3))
 (segment (start 49.99736 37.23894) (end 51.60518 37.23894) (width 0.254) (layer F.Cu) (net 3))
 (segment (start 51.60518 37.23894) (end 51.96078 37.59454) (width 0.254) (layer F.Cu) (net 3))
 (segment (start 51.79314 37.10686) (end 51.66106 37.23894) (width 0.254) (layer F.Cu) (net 3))
 (segment (start 48.6283 32.25038) (end 51.98364 32.25038) (width 0.254) (layer F.Cu) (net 3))
 (segment (start 51.98364 32.25038) (end 51.89728 32.25038) (width 0.254) (layer F.Cu) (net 3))
 (segment (start 47.24908 41.48836) (end 47.24908 42.35958) (width 0.254) (layer F.Cu) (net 3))
 (segment (start 47.49292 41.48836) (end 47.49292 41.3385) (width 0.254) (layer F.Cu) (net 3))
 (segment (start 47.49292 41.3385) (end 47.49292 38.99408) (width 0.254) (layer F.Cu) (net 3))
 (segment (start 47.49292 38.99408) (end 47.498 38.989) (width 0.254) (layer F.Cu) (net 3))
 (segment (start 47.74692 41.48836) (end 47.74692 39.23792) (width 0.254) (layer F.Cu) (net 3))
 (segment (start 47.74692 39.23792) (end 47.498 38.989) (width 0.254) (layer F.Cu) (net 3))
 (segment (start 47.24908 41.48836) (end 47.24908 39.23792) (width 0.254) (layer F.Cu) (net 3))
 (segment (start 47.24908 39.23792) (end 47.498 38.989) (width 0.254) (layer F.Cu) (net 3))
 (segment (start 49.99736 37.23894) (end 49.44364 37.23894) (width 0.254) (layer F.Cu) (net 3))
 (segment (start 47.69358 38.989) (end 47.498 38.989) (width 0.254) (layer F.Cu) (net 3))
 (segment (start 49.44364 37.23894) (end 47.69358 38.989) (width 0.254) (layer F.Cu) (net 3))
 (segment (start 45.68444 33.2994) (end 45.68444 33.54832) (width 0.254) (layer F.Cu) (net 3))
 (segment (start 46.40834 32.5755) (end 45.68444 33.2994) (width 0.254) (layer F.Cu) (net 3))
 (segment (start 46.90364 32.5755) (end 46.40834 32.5755) (width 0.254) (layer F.Cu) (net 3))
 (segment (start 45.68444 33.54832) (end 45.61332 33.61944) (width 0.254) (layer F.Cu) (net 3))
 (segment (start 46.90364 32.5755) (end 47.00778 32.5755) (width 0.254) (layer F.Cu) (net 3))
 (segment (start 49.08606 32.70814) (end 49.08606 33.12424) (width 0.254) (layer F.Cu) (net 3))
 (segment (start 48.68164 32.30372) (end 48.6283 32.25038) (width 0.254) (layer F.Cu) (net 3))
 (segment (start 48.6283 32.25038) (end 49.08606 32.70814) (width 0.254) (layer F.Cu) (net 3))
 (segment (start 47.27956 32.30372) (end 48.68164 32.30372) (width 0.254) (layer F.Cu) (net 3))
 (segment (start 47.00778 32.5755) (end 47.27956 32.30372) (width 0.254) (layer F.Cu) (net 3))
 (segment (start 47.88606 34.72424) (end 47.88606 34.46328) (width 0.254) (layer F.Cu) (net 3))
 (segment (start 49.08606 33.26328) (end 49.08606 33.12424) (width 0.254) (layer F.Cu) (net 3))
 (segment (start 47.88606 34.46328) (end 49.08606 33.26328) (width 0.254) (layer F.Cu) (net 3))
 (segment (start 47.24908 41.48836) (end 47.49292 41.48836) (width 0.254) (layer F.Cu) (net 3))
 (segment (start 47.49292 41.48836) (end 47.74692 41.48836) (width 0.254) (layer F.Cu) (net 3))
 (segment (start 47.74692 36.48964) (end 47.74692 35.8775) (width 0.254) (layer F.Cu) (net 13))
 (segment (start 47.43948 33.12424) (end 47.88606 33.12424) (width 0.254) (layer F.Cu) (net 13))
 (segment (start 47.11446 33.44926) (end 47.43948 33.12424) (width 0.254) (layer F.Cu) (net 13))
 (segment (start 47.11446 35.19678) (end 47.11446 33.44926) (width 0.254) (layer F.Cu) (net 13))
 (segment (start 47.244 35.32632) (end 47.11446 35.19678) (width 0.254) (layer F.Cu) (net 13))
 (segment (start 47.244 35.4965) (end 47.244 35.32632) (width 0.254) (layer F.Cu) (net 13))
 (segment (start 47.41418 35.66668) (end 47.244 35.4965) (width 0.254) (layer F.Cu) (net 13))
 (segment (start 47.5361 35.66668) (end 47.41418 35.66668) (width 0.254) (layer F.Cu) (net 13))
 (segment (start 47.74692 35.8775) (end 47.5361 35.66668) (width 0.254) (layer F.Cu) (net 13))
 (segment (start 44.99864 37.73932) (end 43.71594 37.73932) (width 0.254) (layer F.Cu) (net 5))
 (segment (start 43.71594 37.73932) (end 43.447035 37.470415) (width 0.254) (layer F.Cu) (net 5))
 (segment (start 49.08606 34.72424) (end 49.67234 34.72424) (width 0.254) (layer F.Cu) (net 12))
 (segment (start 49.67234 34.72424) (end 50.038 34.35858) (width 0.254) (layer F.Cu) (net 12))
 (segment (start 48.2473 36.48964) (end 48.2473 35.69462) (width 0.254) (layer F.Cu) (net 12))
 (segment (start 49.08606 34.85586) (end 49.08606 34.72424) (width 0.254) (layer F.Cu) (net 12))
 (segment (start 48.2473 35.69462) (end 49.08606 34.85586) (width 0.254) (layer F.Cu) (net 12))
 (segment (start 46.24832 36.48964) (end 46.24832 35.77844) (width 0.254) (layer F.Cu) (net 7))
 (segment (start 46.24832 35.77844) (end 45.61332 35.14344) (width 0.254) (layer F.Cu) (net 7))
 (segment (start 42.598005 36.341985) (end 42.291 36.03498) (width 0.254) (layer F.Cu) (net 4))
 (segment (start 42.291 36.03498) (end 42.291 35.687) (width 0.254) (layer F.Cu) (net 4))
 (segment (start 44.99864 39.7383) (end 43.73118 39.7383) (width 0.254) (layer F.Cu) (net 8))
 (segment (start 43.73118 39.7383) (end 43.71848 39.7256) (width 0.254) (layer F.Cu) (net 8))
 (segment (start 50.81524 34.74212) (end 51.816 33.74136) (width 0.254) (layer F.Cu) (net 11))
 (segment (start 48.74768 35.91052) (end 49.18456 35.47364) (width 0.254) (layer F.Cu) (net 11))
 (segment (start 49.18456 35.47364) (end 50.08372 35.47364) (width 0.254) (layer F.Cu) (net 11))
 (segment (start 50.08372 35.47364) (end 50.81524 34.74212) (width 0.254) (layer F.Cu) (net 11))
 (segment (start 48.74768 36.48964) (end 48.74768 35.91052) (width 0.254) (layer F.Cu) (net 11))
 (segment (start 51.816 33.74136) (end 51.816 33.528) (width 0.254) (layer F.Cu) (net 11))
 (segment (start 51.89982 35.27552) (end 50.6857 36.48964) (width 0.254) (layer F.Cu) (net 10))
 (segment (start 50.6857 36.48964) (end 49.24806 36.48964) (width 0.254) (layer F.Cu) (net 10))
 (segment (start 51.5874 43.2308) (end 51.5874 42.42816) (width 0.254) (layer F.Cu) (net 6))
 (segment (start 51.5874 42.42816) (end 51.4477 42.28846) (width 0.254) (layer F.Cu) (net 6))
 (segment (start 51.4477 42.28846) (end 48.93564 42.28846) (width 0.254) (layer F.Cu) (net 6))
 (segment (start 48.74768 42.1005) (end 48.74768 41.48836) (width 0.254) (layer F.Cu) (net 6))
 (segment (start 48.93564 42.28846) (end 48.74768 42.1005) (width 0.254) (layer F.Cu) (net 6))
 (segment (start 43.688 41.656) (end 45.5803 41.656) (width 0.254) (layer F.Cu) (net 9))
 (segment (start 45.5803 41.656) (end 45.74794 41.48836) (width 0.254) (layer F.Cu) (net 9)))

